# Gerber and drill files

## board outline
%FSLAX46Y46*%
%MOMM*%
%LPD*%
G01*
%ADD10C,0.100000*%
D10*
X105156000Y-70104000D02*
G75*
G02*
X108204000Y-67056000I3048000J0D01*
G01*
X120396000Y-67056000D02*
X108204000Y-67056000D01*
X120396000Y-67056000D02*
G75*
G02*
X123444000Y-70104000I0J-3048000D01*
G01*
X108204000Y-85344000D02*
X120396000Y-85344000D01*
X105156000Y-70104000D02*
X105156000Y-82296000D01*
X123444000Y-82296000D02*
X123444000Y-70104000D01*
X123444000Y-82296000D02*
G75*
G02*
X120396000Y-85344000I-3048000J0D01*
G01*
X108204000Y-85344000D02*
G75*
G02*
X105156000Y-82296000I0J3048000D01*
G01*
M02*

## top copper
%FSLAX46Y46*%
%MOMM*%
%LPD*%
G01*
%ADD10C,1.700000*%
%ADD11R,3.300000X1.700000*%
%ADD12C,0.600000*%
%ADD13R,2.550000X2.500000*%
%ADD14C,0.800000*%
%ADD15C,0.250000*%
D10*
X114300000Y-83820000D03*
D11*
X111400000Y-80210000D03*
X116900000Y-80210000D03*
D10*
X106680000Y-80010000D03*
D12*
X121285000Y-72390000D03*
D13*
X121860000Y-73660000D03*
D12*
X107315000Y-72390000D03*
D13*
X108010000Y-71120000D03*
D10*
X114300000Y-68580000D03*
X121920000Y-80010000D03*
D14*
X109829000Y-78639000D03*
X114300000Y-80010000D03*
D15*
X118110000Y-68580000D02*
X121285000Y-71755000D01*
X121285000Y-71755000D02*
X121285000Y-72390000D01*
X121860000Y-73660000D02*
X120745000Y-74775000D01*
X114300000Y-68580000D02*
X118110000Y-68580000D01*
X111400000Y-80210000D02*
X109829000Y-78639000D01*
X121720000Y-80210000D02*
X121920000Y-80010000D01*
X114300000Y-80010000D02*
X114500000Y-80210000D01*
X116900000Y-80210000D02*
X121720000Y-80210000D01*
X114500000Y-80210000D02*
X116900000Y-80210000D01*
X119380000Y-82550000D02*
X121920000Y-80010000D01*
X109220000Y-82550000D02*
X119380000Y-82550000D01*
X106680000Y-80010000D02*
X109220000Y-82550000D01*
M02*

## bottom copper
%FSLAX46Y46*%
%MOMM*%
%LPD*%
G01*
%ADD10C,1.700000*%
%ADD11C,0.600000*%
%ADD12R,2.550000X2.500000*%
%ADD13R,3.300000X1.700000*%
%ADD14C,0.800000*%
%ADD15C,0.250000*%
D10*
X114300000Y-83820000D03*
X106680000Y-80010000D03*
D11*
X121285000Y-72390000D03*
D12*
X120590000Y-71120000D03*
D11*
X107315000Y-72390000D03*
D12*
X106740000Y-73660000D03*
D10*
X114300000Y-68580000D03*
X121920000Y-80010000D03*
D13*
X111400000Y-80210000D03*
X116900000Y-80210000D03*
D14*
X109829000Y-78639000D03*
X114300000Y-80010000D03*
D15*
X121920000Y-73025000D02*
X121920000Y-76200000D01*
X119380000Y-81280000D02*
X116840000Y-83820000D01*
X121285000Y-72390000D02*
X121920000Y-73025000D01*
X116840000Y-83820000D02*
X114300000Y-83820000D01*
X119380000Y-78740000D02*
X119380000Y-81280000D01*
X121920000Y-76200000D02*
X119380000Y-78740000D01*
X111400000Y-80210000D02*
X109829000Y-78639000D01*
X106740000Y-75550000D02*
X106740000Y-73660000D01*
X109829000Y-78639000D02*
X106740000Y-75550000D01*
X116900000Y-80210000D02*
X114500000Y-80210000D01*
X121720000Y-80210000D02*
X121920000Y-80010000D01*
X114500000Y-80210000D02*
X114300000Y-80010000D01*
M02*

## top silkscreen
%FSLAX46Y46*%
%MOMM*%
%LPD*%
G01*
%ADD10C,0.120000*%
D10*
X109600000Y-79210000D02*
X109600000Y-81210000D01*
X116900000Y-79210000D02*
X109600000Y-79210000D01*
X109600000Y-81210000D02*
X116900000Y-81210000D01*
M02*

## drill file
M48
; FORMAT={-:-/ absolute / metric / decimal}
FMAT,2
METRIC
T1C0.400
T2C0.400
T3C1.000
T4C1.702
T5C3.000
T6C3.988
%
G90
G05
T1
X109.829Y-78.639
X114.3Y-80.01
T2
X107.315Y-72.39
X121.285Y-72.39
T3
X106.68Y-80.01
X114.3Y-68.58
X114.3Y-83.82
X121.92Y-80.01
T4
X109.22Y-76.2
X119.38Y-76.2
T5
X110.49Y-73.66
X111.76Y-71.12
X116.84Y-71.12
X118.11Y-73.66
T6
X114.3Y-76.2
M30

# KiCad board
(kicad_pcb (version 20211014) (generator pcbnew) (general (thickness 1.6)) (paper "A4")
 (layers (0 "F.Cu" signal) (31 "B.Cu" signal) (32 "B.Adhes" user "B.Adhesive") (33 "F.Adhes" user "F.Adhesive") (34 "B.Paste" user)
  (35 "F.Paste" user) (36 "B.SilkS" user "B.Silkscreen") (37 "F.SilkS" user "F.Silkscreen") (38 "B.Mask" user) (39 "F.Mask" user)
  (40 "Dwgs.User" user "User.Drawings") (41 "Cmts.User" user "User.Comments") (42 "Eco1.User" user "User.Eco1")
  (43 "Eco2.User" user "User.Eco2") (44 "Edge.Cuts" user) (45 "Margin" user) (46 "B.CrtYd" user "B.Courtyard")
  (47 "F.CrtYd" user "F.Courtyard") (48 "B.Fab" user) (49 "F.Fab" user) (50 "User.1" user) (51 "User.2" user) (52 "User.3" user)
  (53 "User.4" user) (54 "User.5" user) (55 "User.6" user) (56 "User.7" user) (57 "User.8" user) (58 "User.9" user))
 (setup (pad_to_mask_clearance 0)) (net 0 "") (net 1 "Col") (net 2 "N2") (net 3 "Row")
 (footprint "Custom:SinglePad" (layer "F.Cu") (at 114.3 83.82)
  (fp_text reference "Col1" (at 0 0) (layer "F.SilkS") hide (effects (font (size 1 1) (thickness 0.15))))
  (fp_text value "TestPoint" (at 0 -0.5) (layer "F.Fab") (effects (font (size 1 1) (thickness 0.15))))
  (pad "1" thru_hole circle locked (at 0 0) (size 1.7 1.7) (drill 1) (layers *.Cu *.Mask) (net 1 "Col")))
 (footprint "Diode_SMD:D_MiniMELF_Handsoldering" (layer "F.Cu") (at 114.15 80.21)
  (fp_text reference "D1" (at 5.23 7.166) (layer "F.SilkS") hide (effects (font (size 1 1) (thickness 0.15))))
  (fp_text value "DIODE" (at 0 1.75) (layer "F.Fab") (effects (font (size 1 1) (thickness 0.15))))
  (fp_line (start -4.55 -1) (end -4.55 1) (layer "F.SilkS") (width 0.12))
  (fp_line (start 2.75 -1) (end -4.55 -1) (layer "F.SilkS") (width 0.12))
  (fp_line (start -4.55 1) (end 2.75 1) (layer "F.SilkS") (width 0.12))
  (pad "1" smd rect (at -2.75 0) (size 3.3 1.7) (layers "F.Cu" "F.Paste" "F.Mask") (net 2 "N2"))
  (pad "2" smd rect (at 2.75 0) (size 3.3 1.7) (layers "F.Cu" "F.Paste" "F.Mask") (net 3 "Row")))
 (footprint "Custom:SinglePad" (layer "F.Cu") (at 106.68 80.01)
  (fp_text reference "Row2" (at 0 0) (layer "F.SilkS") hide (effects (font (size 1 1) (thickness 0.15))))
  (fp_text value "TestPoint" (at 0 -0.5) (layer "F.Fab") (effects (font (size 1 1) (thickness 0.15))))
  (pad "1" thru_hole circle locked (at 0 0) (size 1.7 1.7) (drill 1) (layers *.Cu *.Mask) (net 3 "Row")))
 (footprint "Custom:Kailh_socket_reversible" (layer "F.Cu") (at 114.3 76.2)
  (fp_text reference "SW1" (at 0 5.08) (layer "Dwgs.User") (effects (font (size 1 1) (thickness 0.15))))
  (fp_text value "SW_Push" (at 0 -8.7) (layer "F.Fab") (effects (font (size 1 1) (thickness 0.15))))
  (pad "" np_thru_hole circle (at 2.54 -5.08) (size 3 3) (drill 3) (layers *.Cu *.Mask))
  (pad "" np_thru_hole circle (at 5.08 0) (size 1.7018 1.7018) (drill 1.7018) (layers *.Cu *.Mask))
  (pad "" np_thru_hole circle (at -2.54 -5.08 180) (size 3 3) (drill 3) (layers *.Cu *.Mask))
  (pad "" np_thru_hole circle (at 0 0) (size 3.9878 3.9878) (drill 3.9878) (layers *.Cu *.Mask))
  (pad "" np_thru_hole circle (at 3.81 -2.54 180) (size 3 3) (drill 3) (layers *.Cu *.Mask))
  (pad "" np_thru_hole circle (at -5.08 0) (size 1.7018 1.7018) (drill 1.7018) (layers *.Cu *.Mask))
  (pad "" np_thru_hole circle (at -3.81 -2.54) (size 3 3) (drill 3) (layers *.Cu *.Mask))
  (pad "1" thru_hole circle (at 6.985 -3.81) (size 0.6 0.6) (drill 0.4) (layers *.Cu *.Mask) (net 1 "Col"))
  (pad "1" smd rect (at 7.56 -2.54 180) (size 2.55 2.5) (layers "F.Cu" "F.Paste" "F.Mask") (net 1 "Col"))
  (pad "1" smd rect (at 6.29 -5.08) (size 2.55 2.5) (layers "B.Cu" "B.Paste" "B.Mask") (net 1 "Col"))
  (pad "2" thru_hole circle (at -6.985 -3.81 180) (size 0.6 0.6) (drill 0.4) (layers *.Cu *.Mask) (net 2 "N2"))
  (pad "2" smd rect (at -7.56 -2.54) (size 2.55 2.5) (layers "B.Cu" "B.Paste" "B.Mask") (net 2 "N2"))
  (pad "2" smd rect (at -6.29 -5.08 180) (size 2.55 2.5) (layers "F.Cu" "F.Paste" "F.Mask") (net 2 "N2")))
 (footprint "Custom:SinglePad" (layer "F.Cu") (at 114.3 68.58)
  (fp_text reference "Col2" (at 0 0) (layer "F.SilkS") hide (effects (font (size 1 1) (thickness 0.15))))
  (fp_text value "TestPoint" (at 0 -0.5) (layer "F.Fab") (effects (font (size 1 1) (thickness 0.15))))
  (pad "1" thru_hole circle locked (at 0 0) (size 1.7 1.7) (drill 1) (layers *.Cu *.Mask) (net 1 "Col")))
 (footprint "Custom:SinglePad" (layer "F.Cu") (at 121.92 80.01)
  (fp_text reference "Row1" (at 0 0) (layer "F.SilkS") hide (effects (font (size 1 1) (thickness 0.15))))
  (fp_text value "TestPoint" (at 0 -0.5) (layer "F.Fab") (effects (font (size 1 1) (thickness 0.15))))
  (pad "1" thru_hole circle locked (at 0 0) (size 1.7 1.7) (drill 1) (layers *.Cu *.Mask) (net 3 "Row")))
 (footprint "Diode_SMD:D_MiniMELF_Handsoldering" (layer "B.Cu") (at 114.15 80.21)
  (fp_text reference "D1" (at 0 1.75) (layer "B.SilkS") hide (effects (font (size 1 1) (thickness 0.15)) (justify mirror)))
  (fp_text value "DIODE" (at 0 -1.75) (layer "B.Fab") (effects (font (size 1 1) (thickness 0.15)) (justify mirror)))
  (pad "1" smd rect (at -2.75 0) (size 3.3 1.7) (layers "B.Cu" "B.Paste" "B.Mask") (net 2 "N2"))
  (pad "2" smd rect (at 2.75 0) (size 3.3 1.7) (layers "B.Cu" "B.Paste" "B.Mask") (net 3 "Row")))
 (gr_arc (start 105.156 70.104) (mid 106.048739 67.948739) (end 108.204 67.056) (layer "Edge.Cuts") (width 0.1))
 (gr_line (start 120.396 67.056) (end 108.204 67.056) (layer "Edge.Cuts") (width 0.1))
 (gr_arc (start 120.396 67.056) (mid 122.551261 67.948739) (end 123.444 70.104) (layer "Edge.Cuts") (width 0.1))
 (gr_line (start 108.204 85.344) (end 120.396 85.344) (layer "Edge.Cuts") (width 0.1))
 (gr_line (start 105.156 70.104) (end 105.156 82.296) (layer "Edge.Cuts") (width 0.1))
 (gr_line (start 123.444 82.296) (end 123.444 70.104) (layer "Edge.Cuts") (width 0.1))
 (gr_arc (start 123.444 82.296) (mid 122.551261 84.451261) (end 120.396 85.344) (layer "Edge.Cuts") (width 0.1))
 (gr_arc (start 108.204 85.344) (mid 106.048739 84.451261) (end 105.156 82.296) (layer "Edge.Cuts") (width 0.1))
 (segment (start 118.11 68.58) (end 121.285 71.755) (width 0.25) (layer "F.Cu") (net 1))
 (segment (start 121.285 71.755) (end 121.285 72.39) (width 0.25) (layer "F.Cu") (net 1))
 (segment (start 121.86 73.66) (end 120.745 74.775) (width 0.25) (layer "F.Cu") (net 1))
 (segment (start 114.3 68.58) (end 118.11 68.58) (width 0.25) (layer "F.Cu") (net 1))
 (segment (start 121.92 73.025) (end 121.92 76.2) (width 0.25) (layer "B.Cu") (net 1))
 (segment (start 119.38 81.28) (end 116.84 83.82) (width 0.25) (layer "B.Cu") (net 1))
 (segment (start 121.285 72.39) (end 121.92 73.025) (width 0.25) (layer "B.Cu") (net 1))
 (segment (start 116.84 83.82) (end 114.3 83.82) (width 0.25) (layer "B.Cu") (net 1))
 (segment (start 119.38 78.74) (end 119.38 81.28) (width 0.25) (layer "B.Cu") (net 1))
 (segment (start 121.92 76.2) (end 119.38 78.74) (width 0.25) (layer "B.Cu") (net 1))
 (segment (start 111.4 80.21) (end 109.829 78.639) (width 0.25) (layer "F.Cu") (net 2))
 (via (at 109.829 78.639) (size 0.8) (drill 0.4) (layers "F.Cu" "B.Cu") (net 2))
 (segment (start 111.4 80.21) (end 109.829 78.639) (width 0.25) (layer "B.Cu") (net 2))
 (segment (start 106.74 75.55) (end 106.74 73.66) (width 0.25) (layer "B.Cu") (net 2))
 (segment (start 109.829 78.639) (end 106.74 75.55) (width 0.25) (layer "B.Cu") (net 2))
 (segment (start 121.72 80.21) (end 121.92 80.01) (width 0.25) (layer "F.Cu") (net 3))
 (segment (start 114.3 80.01) (end 114.5 80.21) (width 0.25) (layer "F.Cu") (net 3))
 (segment (start 116.9 80.21) (end 121.72 80.21) (width 0.25) (layer "F.Cu") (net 3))
 (segment (start 114.5 80.21) (end 116.9 80.21) (width 0.25) (layer "F.Cu") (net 3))
 (segment (start 119.38 82.55) (end 121.92 80.01) (width 0.25) (layer "F.Cu") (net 3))
 (segment (start 109.22 82.55) (end 119.38 82.55) (width 0.25) (layer "F.Cu") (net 3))
 (segment (start 106.68 80.01) (end 109.22 82.55) (width 0.25) (layer "F.Cu") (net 3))
 (via (at 114.3 80.01) (size 0.8) (drill 0.4) (layers "F.Cu" "B.Cu") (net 3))
 (segment (start 116.9 80.21) (end 114.5 80.21) (width 0.25) (layer "B.Cu") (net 3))
 (segment (start 121.72 80.21) (end 121.92 80.01) (width 0.25) (layer "B.Cu") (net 3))
 (segment (start 114.5 80.21) (end 114.3 80.01) (width 0.25) (layer "B.Cu") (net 3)))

